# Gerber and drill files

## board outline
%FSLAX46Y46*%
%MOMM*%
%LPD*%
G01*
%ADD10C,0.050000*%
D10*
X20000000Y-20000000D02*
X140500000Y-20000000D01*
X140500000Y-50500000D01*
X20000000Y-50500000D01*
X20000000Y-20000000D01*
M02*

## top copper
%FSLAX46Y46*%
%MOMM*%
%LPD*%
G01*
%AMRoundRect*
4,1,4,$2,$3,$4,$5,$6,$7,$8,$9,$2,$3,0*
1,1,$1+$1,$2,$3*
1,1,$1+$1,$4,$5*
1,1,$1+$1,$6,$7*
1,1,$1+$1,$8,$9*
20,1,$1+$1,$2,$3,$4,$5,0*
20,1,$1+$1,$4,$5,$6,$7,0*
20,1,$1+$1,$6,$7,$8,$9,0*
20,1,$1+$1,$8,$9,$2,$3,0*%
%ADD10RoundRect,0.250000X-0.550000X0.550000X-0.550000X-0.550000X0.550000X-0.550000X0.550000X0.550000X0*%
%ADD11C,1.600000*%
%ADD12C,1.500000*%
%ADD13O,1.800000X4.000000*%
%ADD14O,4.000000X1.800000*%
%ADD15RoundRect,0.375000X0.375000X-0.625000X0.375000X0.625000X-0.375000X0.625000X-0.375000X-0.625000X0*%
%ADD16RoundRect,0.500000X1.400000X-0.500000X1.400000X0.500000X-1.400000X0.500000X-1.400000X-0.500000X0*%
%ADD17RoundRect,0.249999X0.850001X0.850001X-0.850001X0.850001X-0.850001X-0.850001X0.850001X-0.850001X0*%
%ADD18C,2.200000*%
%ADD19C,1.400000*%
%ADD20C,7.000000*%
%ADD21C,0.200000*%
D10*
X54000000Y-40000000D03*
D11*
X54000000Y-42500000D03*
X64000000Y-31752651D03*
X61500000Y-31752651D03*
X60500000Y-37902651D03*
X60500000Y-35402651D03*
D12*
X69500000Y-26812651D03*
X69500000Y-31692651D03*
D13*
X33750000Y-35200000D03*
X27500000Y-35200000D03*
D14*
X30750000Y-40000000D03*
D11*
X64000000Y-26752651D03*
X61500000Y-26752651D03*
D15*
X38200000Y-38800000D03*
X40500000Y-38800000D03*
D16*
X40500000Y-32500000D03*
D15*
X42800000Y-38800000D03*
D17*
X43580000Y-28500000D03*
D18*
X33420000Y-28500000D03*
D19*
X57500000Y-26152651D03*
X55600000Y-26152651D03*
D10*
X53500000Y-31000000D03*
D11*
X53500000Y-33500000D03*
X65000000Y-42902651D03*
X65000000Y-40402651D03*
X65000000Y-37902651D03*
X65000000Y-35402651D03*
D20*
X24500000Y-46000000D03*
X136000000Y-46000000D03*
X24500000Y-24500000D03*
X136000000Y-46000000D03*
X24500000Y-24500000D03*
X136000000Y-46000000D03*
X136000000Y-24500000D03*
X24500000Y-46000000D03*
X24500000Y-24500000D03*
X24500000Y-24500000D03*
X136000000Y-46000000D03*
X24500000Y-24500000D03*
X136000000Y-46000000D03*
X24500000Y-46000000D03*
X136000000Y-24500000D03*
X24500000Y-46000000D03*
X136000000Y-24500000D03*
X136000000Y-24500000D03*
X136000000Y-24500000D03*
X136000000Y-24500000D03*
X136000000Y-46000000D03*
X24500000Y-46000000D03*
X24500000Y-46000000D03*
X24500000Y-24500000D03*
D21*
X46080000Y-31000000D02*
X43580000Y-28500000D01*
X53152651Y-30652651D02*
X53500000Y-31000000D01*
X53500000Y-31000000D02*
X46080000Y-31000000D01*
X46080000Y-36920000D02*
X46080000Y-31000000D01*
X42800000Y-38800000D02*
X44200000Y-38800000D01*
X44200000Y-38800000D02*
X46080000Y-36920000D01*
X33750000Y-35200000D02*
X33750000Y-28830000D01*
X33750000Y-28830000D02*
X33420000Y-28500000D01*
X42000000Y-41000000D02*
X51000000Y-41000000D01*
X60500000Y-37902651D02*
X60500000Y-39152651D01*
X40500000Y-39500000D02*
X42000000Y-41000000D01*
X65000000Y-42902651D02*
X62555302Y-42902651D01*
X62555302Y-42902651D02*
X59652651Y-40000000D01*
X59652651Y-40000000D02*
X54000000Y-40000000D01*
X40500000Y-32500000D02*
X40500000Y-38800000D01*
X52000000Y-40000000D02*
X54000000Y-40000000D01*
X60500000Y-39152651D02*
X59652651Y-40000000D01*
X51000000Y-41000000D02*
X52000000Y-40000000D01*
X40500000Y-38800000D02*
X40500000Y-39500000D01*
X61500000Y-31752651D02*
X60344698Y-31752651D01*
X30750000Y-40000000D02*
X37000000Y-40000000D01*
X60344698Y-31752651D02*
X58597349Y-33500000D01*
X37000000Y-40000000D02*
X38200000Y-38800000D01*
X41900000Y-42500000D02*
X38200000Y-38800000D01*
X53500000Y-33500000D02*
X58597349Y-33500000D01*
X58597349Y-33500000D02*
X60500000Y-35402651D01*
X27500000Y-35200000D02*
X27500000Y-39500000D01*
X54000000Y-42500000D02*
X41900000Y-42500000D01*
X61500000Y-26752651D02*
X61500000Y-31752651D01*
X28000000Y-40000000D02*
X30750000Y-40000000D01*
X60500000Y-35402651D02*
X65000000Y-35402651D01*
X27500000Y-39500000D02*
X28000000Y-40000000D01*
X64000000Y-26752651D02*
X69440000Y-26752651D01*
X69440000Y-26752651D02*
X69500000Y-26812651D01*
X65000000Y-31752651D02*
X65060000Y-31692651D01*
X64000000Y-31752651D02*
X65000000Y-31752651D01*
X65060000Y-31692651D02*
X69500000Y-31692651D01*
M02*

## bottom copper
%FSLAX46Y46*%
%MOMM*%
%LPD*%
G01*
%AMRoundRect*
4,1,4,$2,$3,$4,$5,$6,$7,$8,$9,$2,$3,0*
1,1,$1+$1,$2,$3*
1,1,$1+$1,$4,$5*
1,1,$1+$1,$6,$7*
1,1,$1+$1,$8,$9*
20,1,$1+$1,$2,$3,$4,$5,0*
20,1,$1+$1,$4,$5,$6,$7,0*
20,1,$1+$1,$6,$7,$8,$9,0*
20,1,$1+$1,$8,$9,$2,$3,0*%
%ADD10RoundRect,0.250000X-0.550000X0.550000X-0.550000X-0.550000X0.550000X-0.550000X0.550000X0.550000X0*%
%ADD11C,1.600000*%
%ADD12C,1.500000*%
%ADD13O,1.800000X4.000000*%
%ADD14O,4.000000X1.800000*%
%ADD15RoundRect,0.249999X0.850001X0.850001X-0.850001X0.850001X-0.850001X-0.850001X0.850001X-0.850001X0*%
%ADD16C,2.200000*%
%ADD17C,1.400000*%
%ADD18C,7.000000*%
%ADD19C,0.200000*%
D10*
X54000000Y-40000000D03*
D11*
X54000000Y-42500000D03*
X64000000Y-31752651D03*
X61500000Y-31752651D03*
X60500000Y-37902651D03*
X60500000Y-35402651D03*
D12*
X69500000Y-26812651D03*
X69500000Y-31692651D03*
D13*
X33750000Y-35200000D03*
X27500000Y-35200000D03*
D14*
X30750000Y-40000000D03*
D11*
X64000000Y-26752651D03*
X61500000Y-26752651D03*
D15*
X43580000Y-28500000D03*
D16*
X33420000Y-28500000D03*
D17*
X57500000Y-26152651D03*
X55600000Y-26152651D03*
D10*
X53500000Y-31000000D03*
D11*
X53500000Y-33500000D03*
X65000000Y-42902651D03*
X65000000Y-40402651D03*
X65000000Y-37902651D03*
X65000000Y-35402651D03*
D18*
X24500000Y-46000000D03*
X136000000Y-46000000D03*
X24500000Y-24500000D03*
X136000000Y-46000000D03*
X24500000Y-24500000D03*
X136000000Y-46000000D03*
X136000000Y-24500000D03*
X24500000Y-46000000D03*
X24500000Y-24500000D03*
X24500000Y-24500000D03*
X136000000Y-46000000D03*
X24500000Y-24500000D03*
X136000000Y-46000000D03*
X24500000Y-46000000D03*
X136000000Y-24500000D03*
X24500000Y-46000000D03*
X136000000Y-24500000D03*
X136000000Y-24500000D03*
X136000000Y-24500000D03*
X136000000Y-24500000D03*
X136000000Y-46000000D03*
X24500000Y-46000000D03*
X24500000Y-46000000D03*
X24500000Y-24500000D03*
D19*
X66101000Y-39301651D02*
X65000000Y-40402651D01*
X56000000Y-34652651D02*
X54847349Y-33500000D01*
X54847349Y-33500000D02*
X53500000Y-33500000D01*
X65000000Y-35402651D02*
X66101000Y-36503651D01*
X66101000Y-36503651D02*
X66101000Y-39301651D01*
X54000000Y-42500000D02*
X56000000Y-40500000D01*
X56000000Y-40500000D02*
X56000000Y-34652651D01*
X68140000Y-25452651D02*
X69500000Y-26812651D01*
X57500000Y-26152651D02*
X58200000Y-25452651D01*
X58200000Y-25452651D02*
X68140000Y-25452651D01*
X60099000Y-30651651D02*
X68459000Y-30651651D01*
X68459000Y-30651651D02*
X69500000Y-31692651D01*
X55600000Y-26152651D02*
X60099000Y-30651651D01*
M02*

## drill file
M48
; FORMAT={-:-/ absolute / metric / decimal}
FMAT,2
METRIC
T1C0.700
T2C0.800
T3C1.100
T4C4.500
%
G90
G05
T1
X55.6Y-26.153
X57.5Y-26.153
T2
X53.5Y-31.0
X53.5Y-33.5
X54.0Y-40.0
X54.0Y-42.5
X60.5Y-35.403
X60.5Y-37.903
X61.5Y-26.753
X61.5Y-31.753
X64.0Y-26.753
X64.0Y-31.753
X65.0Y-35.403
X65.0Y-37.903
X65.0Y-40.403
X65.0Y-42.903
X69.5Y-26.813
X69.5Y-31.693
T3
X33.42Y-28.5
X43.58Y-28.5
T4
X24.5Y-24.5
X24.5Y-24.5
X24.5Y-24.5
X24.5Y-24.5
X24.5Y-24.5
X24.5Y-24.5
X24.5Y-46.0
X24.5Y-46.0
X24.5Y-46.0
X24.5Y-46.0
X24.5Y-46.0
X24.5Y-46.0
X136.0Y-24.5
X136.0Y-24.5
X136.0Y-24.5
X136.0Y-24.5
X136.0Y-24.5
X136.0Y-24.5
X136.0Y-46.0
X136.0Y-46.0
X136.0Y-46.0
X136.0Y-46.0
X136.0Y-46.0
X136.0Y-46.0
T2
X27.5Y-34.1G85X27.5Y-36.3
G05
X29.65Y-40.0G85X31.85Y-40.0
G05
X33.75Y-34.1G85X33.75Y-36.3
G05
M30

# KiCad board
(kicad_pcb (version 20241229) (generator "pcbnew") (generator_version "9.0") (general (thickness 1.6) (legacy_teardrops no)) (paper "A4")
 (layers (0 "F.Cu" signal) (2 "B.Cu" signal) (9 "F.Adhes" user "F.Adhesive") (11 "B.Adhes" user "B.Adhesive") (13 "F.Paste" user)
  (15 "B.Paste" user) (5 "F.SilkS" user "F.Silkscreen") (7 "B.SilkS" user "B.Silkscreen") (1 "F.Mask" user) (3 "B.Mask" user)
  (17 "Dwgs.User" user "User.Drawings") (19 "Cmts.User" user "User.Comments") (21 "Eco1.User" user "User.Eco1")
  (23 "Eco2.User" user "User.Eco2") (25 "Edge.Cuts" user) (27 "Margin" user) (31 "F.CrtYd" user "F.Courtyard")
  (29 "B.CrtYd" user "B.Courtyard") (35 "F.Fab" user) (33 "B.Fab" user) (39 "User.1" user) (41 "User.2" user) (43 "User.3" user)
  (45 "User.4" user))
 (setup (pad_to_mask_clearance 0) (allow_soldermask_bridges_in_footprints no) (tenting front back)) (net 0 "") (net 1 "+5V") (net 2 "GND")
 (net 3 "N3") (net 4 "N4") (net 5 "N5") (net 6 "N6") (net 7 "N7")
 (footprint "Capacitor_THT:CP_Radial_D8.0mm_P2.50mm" (layer "F.Cu") (at 54 40 -90)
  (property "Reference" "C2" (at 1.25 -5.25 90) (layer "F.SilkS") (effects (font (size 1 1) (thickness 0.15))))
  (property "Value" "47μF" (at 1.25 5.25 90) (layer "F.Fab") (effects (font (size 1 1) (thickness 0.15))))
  (pad "1" thru_hole roundrect (at 0 0 270) (size 1.6 1.6) (drill 0.8) (layers "*.Cu" "*.Mask") (remove_unused_layers no)
   (roundrect_rratio 0.15625) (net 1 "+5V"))
  (pad "2" thru_hole circle (at 2.5 0 270) (size 1.6 1.6) (drill 0.8) (layers "*.Cu" "*.Mask") (remove_unused_layers no) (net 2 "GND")))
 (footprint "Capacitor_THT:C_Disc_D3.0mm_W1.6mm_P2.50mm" (layer "F.Cu") (at 64 31.752651 180)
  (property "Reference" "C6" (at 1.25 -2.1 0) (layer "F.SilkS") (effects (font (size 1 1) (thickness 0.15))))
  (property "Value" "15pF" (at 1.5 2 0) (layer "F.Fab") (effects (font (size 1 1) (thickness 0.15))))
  (pad "1" thru_hole circle (at 0 0 180) (size 1.6 1.6) (drill 0.8) (layers "*.Cu" "*.Mask") (remove_unused_layers no) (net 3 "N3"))
  (pad "2" thru_hole circle (at 2.5 0 180) (size 1.6 1.6) (drill 0.8) (layers "*.Cu" "*.Mask") (remove_unused_layers no) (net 2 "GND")))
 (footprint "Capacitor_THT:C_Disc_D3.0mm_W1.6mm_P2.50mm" (layer "F.Cu") (at 60.5 37.902651 90)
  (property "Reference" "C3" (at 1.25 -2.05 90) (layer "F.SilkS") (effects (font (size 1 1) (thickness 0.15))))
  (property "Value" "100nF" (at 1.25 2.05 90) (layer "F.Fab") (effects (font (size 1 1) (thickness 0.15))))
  (pad "1" thru_hole circle (at 0 0 90) (size 1.6 1.6) (drill 0.8) (layers "*.Cu" "*.Mask") (remove_unused_layers no) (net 1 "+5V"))
  (pad "2" thru_hole circle (at 2.5 0 90) (size 1.6 1.6) (drill 0.8) (layers "*.Cu" "*.Mask") (remove_unused_layers no) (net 2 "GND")))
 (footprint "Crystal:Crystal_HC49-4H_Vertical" (layer "F.Cu") (at 69.5 26.812651 -90)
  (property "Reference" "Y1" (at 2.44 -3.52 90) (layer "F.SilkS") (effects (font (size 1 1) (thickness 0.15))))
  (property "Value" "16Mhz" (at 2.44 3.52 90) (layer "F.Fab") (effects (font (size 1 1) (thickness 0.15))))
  (pad "1" thru_hole circle (at 0 0 270) (size 1.5 1.5) (drill 0.8) (layers "*.Cu" "*.Mask") (remove_unused_layers no) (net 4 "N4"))
  (pad "2" thru_hole circle (at 4.88 0 270) (size 1.5 1.5) (drill 0.8) (layers "*.Cu" "*.Mask") (remove_unused_layers no) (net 3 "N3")))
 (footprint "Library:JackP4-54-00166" (layer "F.Cu") (at 27 35.2)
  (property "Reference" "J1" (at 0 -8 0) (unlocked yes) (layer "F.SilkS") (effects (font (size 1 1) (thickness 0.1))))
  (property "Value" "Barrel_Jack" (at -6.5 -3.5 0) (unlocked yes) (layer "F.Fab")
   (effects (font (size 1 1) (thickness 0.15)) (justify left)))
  (pad "1" thru_hole oval (at 6.75 0) (size 1.8 4) (drill oval 0.8 3) (layers "*.Cu" "*.Mask") (remove_unused_layers no) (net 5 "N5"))
  (pad "2" thru_hole oval (at 0.5 0) (size 1.8 4) (drill oval 0.8 3) (layers "*.Cu" "*.Mask") (remove_unused_layers no) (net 2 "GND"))
  (pad "3" thru_hole oval (at 3.75 4.8 90) (size 1.8 4) (drill oval 0.8 3) (layers "*.Cu" "*.Mask") (remove_unused_layers no) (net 2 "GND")))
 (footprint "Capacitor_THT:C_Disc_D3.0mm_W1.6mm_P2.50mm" (layer "F.Cu") (at 64 26.752651 180)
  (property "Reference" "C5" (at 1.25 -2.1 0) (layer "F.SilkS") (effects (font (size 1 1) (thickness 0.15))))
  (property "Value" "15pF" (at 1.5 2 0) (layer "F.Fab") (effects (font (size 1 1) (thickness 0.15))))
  (pad "1" thru_hole circle (at 0 0 180) (size 1.6 1.6) (drill 0.8) (layers "*.Cu" "*.Mask") (remove_unused_layers no) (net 4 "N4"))
  (pad "2" thru_hole circle (at 2.5 0 180) (size 1.6 1.6) (drill 0.8) (layers "*.Cu" "*.Mask") (remove_unused_layers no) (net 2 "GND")))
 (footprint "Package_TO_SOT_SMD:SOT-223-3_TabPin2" (layer "F.Cu") (at 40.5 35.65 90)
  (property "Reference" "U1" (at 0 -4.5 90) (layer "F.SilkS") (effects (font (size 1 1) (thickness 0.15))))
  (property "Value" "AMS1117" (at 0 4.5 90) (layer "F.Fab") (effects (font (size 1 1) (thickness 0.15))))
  (pad "1" smd roundrect (at -3.15 -2.3 90) (size 2 1.5) (layers "F.Cu" "F.Mask" "F.Paste") (roundrect_rratio 0.25) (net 2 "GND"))
  (pad "2" smd roundrect (at -3.15 0 90) (size 2 1.5) (layers "F.Cu" "F.Mask" "F.Paste") (roundrect_rratio 0.25) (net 1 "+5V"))
  (pad "2" smd roundrect (at 3.15 0 90) (size 2 3.8) (layers "F.Cu" "F.Mask" "F.Paste") (roundrect_rratio 0.25) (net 1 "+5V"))
  (pad "3" smd roundrect (at -3.15 2.3 90) (size 2 1.5) (layers "F.Cu" "F.Mask" "F.Paste") (roundrect_rratio 0.25) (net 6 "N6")))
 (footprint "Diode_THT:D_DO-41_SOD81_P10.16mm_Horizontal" (layer "F.Cu") (at 43.58 28.5 180)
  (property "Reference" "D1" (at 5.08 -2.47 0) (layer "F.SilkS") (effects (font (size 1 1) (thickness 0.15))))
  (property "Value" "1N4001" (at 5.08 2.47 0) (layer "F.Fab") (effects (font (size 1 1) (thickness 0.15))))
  (pad "1" thru_hole roundrect (at 0 0 180) (size 2.2 2.2) (drill 1.1) (layers "*.Cu" "*.Mask") (remove_unused_layers no)
   (roundrect_rratio 0.113636) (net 6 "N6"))
  (pad "2" thru_hole circle (at 10.16 0 180) (size 2.2 2.2) (drill 1.1) (layers "*.Cu" "*.Mask") (remove_unused_layers no) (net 5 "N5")))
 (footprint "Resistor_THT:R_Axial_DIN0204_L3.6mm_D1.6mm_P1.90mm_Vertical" (layer "F.Cu") (at 57.5 26.152651 180)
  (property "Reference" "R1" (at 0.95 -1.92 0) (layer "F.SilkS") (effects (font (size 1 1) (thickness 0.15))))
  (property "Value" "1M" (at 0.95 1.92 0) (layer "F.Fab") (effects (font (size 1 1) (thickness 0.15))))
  (pad "1" thru_hole circle (at 0 0 180) (size 1.4 1.4) (drill 0.7) (layers "*.Cu" "*.Mask") (remove_unused_layers no) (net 4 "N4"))
  (pad "2" thru_hole circle (at 1.9 0 180) (size 1.4 1.4) (drill 0.7) (layers "*.Cu" "*.Mask") (remove_unused_layers no) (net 3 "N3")))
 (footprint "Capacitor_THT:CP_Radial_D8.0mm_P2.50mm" (layer "F.Cu") (at 53.5 31 -90)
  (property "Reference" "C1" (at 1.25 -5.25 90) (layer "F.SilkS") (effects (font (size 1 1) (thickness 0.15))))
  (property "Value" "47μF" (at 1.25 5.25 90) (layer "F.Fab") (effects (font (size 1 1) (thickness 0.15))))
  (pad "1" thru_hole roundrect (at 0 0 270) (size 1.6 1.6) (drill 0.8) (layers "*.Cu" "*.Mask") (remove_unused_layers no)
   (roundrect_rratio 0.15625) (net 6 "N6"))
  (pad "2" thru_hole circle (at 2.5 0 270) (size 1.6 1.6) (drill 0.8) (layers "*.Cu" "*.Mask") (remove_unused_layers no) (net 2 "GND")))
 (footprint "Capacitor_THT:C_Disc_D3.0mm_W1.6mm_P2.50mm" (layer "F.Cu") (at 65 42.902651 90)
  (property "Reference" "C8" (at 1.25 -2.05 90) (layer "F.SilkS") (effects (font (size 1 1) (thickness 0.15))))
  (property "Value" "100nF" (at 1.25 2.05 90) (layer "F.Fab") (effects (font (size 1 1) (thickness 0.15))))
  (pad "1" thru_hole circle (at 0 0 90) (size 1.6 1.6) (drill 0.8) (layers "*.Cu" "*.Mask") (remove_unused_layers no) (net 1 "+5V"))
  (pad "2" thru_hole circle (at 2.5 0 90) (size 1.6 1.6) (drill 0.8) (layers "*.Cu" "*.Mask") (remove_unused_layers no) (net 2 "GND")))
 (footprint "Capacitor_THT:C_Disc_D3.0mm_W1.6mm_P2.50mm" (layer "F.Cu") (at 65 37.902651 90)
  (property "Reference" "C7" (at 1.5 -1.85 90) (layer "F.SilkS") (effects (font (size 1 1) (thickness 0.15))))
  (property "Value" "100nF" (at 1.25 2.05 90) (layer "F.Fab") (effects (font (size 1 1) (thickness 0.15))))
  (pad "1" thru_hole circle (at 0 0 90) (size 1.6 1.6) (drill 0.8) (layers "*.Cu" "*.Mask") (remove_unused_layers no) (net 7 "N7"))
  (pad "2" thru_hole circle (at 2.5 0 90) (size 1.6 1.6) (drill 0.8) (layers "*.Cu" "*.Mask") (remove_unused_layers no) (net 2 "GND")))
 (gr_rect (start 20 20) (end 140.5 50.5) (stroke (width 0.05) (type solid)) (fill no) (layer "Edge.Cuts"))
 (via (at 24.5 46) (size 7) (drill 4.5) (layers "F.Cu" "B.Cu") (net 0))
 (via (at 136 46) (size 7) (drill 4.5) (layers "F.Cu" "B.Cu") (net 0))
 (via (at 24.5 24.5) (size 7) (drill 4.5) (layers "F.Cu" "B.Cu") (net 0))
 (via (at 136 46) (size 7) (drill 4.5) (layers "F.Cu" "B.Cu") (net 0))
 (via (at 24.5 24.5) (size 7) (drill 4.5) (layers "F.Cu" "B.Cu") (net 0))
 (via (at 136 46) (size 7) (drill 4.5) (layers "F.Cu" "B.Cu") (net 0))
 (via (at 136 24.5) (size 7) (drill 4.5) (layers "F.Cu" "B.Cu") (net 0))
 (via (at 24.5 46) (size 7) (drill 4.5) (layers "F.Cu" "B.Cu") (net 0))
 (via (at 24.5 24.5) (size 7) (drill 4.5) (layers "F.Cu" "B.Cu") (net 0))
 (via (at 24.5 24.5) (size 7) (drill 4.5) (layers "F.Cu" "B.Cu") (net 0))
 (via (at 136 46) (size 7) (drill 4.5) (layers "F.Cu" "B.Cu") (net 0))
 (via (at 24.5 24.5) (size 7) (drill 4.5) (layers "F.Cu" "B.Cu") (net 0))
 (via (at 136 46) (size 7) (drill 4.5) (layers "F.Cu" "B.Cu") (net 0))
 (via (at 24.5 46) (size 7) (drill 4.5) (layers "F.Cu" "B.Cu") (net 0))
 (via (at 136 24.5) (size 7) (drill 4.5) (layers "F.Cu" "B.Cu") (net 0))
 (via (at 24.5 46) (size 7) (drill 4.5) (layers "F.Cu" "B.Cu") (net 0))
 (via (at 136 24.5) (size 7) (drill 4.5) (layers "F.Cu" "B.Cu") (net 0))
 (via (at 136 24.5) (size 7) (drill 4.5) (layers "F.Cu" "B.Cu") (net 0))
 (via (at 136 24.5) (size 7) (drill 4.5) (layers "F.Cu" "B.Cu") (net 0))
 (via (at 136 24.5) (size 7) (drill 4.5) (layers "F.Cu" "B.Cu") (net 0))
 (via (at 136 46) (size 7) (drill 4.5) (layers "F.Cu" "B.Cu") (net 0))
 (via (at 24.5 46) (size 7) (drill 4.5) (layers "F.Cu" "B.Cu") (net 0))
 (via (at 24.5 46) (size 7) (drill 4.5) (layers "F.Cu" "B.Cu") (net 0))
 (via (at 24.5 24.5) (size 7) (drill 4.5) (layers "F.Cu" "B.Cu") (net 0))
 (segment (start 46.08 31) (end 43.58 28.5) (width 0.2) (layer "F.Cu") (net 6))
 (segment (start 53.152651 30.652651) (end 53.5 31) (width 0.2) (layer "F.Cu") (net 6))
 (segment (start 53.5 31) (end 46.08 31) (width 0.2) (layer "F.Cu") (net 6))
 (segment (start 46.08 36.92) (end 46.08 31) (width 0.2) (layer "F.Cu") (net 6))
 (segment (start 42.8 38.8) (end 44.2 38.8) (width 0.2) (layer "F.Cu") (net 6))
 (segment (start 44.2 38.8) (end 46.08 36.92) (width 0.2) (layer "F.Cu") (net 6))
 (segment (start 33.75 35.2) (end 33.75 28.83) (width 0.2) (layer "F.Cu") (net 5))
 (segment (start 33.75 28.83) (end 33.42 28.5) (width 0.2) (layer "F.Cu") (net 5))
 (segment (start 42 41) (end 51 41) (width 0.2) (layer "F.Cu") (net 1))
 (segment (start 60.5 37.902651) (end 60.5 39.152651) (width 0.2) (layer "F.Cu") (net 1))
 (segment (start 40.5 39.5) (end 42 41) (width 0.2) (layer "F.Cu") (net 1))
 (segment (start 65 42.902651) (end 62.555302 42.902651) (width 0.2) (layer "F.Cu") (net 1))
 (segment (start 62.555302 42.902651) (end 59.652651 40) (width 0.2) (layer "F.Cu") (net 1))
 (segment (start 59.652651 40) (end 54 40) (width 0.2) (layer "F.Cu") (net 1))
 (segment (start 40.5 32.5) (end 40.5 38.8) (width 0.2) (layer "F.Cu") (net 1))
 (segment (start 52 40) (end 54 40) (width 0.2) (layer "F.Cu") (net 1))
 (segment (start 60.5 39.152651) (end 59.652651 40) (width 0.2) (layer "F.Cu") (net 1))
 (segment (start 51 41) (end 52 40) (width 0.2) (layer "F.Cu") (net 1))
 (segment (start 40.5 38.8) (end 40.5 39.5) (width 0.2) (layer "F.Cu") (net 1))
 (segment (start 61.5 31.752651) (end 60.344698 31.752651) (width 0.2) (layer "F.Cu") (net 2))
 (segment (start 30.75 40) (end 37 40) (width 0.2) (layer "F.Cu") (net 2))
 (segment (start 60.344698 31.752651) (end 58.597349 33.5) (width 0.2) (layer "F.Cu") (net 2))
 (segment (start 37 40) (end 38.2 38.8) (width 0.2) (layer "F.Cu") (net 2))
 (segment (start 41.9 42.5) (end 38.2 38.8) (width 0.2) (layer "F.Cu") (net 2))
 (segment (start 53.5 33.5) (end 58.597349 33.5) (width 0.2) (layer "F.Cu") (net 2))
 (segment (start 58.597349 33.5) (end 60.5 35.402651) (width 0.2) (layer "F.Cu") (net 2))
 (segment (start 27.5 35.2) (end 27.5 39.5) (width 0.2) (layer "F.Cu") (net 2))
 (segment (start 54 42.5) (end 41.9 42.5) (width 0.2) (layer "F.Cu") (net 2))
 (segment (start 61.5 26.752651) (end 61.5 31.752651) (width 0.2) (layer "F.Cu") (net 2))
 (segment (start 28 40) (end 30.75 40) (width 0.2) (layer "F.Cu") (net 2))
 (segment (start 60.5 35.402651) (end 65 35.402651) (width 0.2) (layer "F.Cu") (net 2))
 (segment (start 27.5 39.5) (end 28 40) (width 0.2) (layer "F.Cu") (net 2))
 (segment (start 66.101 39.301651) (end 65 40.402651) (width 0.2) (layer "B.Cu") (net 2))
 (segment (start 56 34.652651) (end 54.847349 33.5) (width 0.2) (layer "B.Cu") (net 2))
 (segment (start 54.847349 33.5) (end 53.5 33.5) (width 0.2) (layer "B.Cu") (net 2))
 (segment (start 65 35.402651) (end 66.101 36.503651) (width 0.2) (layer "B.Cu") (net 2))
 (segment (start 66.101 36.503651) (end 66.101 39.301651) (width 0.2) (layer "B.Cu") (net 2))
 (segment (start 54 42.5) (end 56 40.5) (width 0.2) (layer "B.Cu") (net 2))
 (segment (start 56 40.5) (end 56 34.652651) (width 0.2) (layer "B.Cu") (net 2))
 (segment (start 64 26.752651) (end 69.44 26.752651) (width 0.2) (layer "F.Cu") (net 4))
 (segment (start 69.44 26.752651) (end 69.5 26.812651) (width 0.2) (layer "F.Cu") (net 4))
 (segment (start 68.14 25.452651) (end 69.5 26.812651) (width 0.2) (layer "B.Cu") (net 4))
 (segment (start 57.5 26.152651) (end 58.2 25.452651) (width 0.2) (layer "B.Cu") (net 4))
 (segment (start 58.2 25.452651) (end 68.14 25.452651) (width 0.2) (layer "B.Cu") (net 4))
 (segment (start 65 31.752651) (end 65.06 31.692651) (width 0.2) (layer "F.Cu") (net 3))
 (segment (start 64 31.752651) (end 65 31.752651) (width 0.2) (layer "F.Cu") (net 3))
 (segment (start 65.06 31.692651) (end 69.5 31.692651) (width 0.2) (layer "F.Cu") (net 3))
 (segment (start 60.099 30.651651) (end 68.459 30.651651) (width 0.2) (layer "B.Cu") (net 3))
 (segment (start 68.459 30.651651) (end 69.5 31.692651) (width 0.2) (layer "B.Cu") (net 3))
 (segment (start 55.6 26.152651) (end 60.099 30.651651) (width 0.2) (layer "B.Cu") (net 3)))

